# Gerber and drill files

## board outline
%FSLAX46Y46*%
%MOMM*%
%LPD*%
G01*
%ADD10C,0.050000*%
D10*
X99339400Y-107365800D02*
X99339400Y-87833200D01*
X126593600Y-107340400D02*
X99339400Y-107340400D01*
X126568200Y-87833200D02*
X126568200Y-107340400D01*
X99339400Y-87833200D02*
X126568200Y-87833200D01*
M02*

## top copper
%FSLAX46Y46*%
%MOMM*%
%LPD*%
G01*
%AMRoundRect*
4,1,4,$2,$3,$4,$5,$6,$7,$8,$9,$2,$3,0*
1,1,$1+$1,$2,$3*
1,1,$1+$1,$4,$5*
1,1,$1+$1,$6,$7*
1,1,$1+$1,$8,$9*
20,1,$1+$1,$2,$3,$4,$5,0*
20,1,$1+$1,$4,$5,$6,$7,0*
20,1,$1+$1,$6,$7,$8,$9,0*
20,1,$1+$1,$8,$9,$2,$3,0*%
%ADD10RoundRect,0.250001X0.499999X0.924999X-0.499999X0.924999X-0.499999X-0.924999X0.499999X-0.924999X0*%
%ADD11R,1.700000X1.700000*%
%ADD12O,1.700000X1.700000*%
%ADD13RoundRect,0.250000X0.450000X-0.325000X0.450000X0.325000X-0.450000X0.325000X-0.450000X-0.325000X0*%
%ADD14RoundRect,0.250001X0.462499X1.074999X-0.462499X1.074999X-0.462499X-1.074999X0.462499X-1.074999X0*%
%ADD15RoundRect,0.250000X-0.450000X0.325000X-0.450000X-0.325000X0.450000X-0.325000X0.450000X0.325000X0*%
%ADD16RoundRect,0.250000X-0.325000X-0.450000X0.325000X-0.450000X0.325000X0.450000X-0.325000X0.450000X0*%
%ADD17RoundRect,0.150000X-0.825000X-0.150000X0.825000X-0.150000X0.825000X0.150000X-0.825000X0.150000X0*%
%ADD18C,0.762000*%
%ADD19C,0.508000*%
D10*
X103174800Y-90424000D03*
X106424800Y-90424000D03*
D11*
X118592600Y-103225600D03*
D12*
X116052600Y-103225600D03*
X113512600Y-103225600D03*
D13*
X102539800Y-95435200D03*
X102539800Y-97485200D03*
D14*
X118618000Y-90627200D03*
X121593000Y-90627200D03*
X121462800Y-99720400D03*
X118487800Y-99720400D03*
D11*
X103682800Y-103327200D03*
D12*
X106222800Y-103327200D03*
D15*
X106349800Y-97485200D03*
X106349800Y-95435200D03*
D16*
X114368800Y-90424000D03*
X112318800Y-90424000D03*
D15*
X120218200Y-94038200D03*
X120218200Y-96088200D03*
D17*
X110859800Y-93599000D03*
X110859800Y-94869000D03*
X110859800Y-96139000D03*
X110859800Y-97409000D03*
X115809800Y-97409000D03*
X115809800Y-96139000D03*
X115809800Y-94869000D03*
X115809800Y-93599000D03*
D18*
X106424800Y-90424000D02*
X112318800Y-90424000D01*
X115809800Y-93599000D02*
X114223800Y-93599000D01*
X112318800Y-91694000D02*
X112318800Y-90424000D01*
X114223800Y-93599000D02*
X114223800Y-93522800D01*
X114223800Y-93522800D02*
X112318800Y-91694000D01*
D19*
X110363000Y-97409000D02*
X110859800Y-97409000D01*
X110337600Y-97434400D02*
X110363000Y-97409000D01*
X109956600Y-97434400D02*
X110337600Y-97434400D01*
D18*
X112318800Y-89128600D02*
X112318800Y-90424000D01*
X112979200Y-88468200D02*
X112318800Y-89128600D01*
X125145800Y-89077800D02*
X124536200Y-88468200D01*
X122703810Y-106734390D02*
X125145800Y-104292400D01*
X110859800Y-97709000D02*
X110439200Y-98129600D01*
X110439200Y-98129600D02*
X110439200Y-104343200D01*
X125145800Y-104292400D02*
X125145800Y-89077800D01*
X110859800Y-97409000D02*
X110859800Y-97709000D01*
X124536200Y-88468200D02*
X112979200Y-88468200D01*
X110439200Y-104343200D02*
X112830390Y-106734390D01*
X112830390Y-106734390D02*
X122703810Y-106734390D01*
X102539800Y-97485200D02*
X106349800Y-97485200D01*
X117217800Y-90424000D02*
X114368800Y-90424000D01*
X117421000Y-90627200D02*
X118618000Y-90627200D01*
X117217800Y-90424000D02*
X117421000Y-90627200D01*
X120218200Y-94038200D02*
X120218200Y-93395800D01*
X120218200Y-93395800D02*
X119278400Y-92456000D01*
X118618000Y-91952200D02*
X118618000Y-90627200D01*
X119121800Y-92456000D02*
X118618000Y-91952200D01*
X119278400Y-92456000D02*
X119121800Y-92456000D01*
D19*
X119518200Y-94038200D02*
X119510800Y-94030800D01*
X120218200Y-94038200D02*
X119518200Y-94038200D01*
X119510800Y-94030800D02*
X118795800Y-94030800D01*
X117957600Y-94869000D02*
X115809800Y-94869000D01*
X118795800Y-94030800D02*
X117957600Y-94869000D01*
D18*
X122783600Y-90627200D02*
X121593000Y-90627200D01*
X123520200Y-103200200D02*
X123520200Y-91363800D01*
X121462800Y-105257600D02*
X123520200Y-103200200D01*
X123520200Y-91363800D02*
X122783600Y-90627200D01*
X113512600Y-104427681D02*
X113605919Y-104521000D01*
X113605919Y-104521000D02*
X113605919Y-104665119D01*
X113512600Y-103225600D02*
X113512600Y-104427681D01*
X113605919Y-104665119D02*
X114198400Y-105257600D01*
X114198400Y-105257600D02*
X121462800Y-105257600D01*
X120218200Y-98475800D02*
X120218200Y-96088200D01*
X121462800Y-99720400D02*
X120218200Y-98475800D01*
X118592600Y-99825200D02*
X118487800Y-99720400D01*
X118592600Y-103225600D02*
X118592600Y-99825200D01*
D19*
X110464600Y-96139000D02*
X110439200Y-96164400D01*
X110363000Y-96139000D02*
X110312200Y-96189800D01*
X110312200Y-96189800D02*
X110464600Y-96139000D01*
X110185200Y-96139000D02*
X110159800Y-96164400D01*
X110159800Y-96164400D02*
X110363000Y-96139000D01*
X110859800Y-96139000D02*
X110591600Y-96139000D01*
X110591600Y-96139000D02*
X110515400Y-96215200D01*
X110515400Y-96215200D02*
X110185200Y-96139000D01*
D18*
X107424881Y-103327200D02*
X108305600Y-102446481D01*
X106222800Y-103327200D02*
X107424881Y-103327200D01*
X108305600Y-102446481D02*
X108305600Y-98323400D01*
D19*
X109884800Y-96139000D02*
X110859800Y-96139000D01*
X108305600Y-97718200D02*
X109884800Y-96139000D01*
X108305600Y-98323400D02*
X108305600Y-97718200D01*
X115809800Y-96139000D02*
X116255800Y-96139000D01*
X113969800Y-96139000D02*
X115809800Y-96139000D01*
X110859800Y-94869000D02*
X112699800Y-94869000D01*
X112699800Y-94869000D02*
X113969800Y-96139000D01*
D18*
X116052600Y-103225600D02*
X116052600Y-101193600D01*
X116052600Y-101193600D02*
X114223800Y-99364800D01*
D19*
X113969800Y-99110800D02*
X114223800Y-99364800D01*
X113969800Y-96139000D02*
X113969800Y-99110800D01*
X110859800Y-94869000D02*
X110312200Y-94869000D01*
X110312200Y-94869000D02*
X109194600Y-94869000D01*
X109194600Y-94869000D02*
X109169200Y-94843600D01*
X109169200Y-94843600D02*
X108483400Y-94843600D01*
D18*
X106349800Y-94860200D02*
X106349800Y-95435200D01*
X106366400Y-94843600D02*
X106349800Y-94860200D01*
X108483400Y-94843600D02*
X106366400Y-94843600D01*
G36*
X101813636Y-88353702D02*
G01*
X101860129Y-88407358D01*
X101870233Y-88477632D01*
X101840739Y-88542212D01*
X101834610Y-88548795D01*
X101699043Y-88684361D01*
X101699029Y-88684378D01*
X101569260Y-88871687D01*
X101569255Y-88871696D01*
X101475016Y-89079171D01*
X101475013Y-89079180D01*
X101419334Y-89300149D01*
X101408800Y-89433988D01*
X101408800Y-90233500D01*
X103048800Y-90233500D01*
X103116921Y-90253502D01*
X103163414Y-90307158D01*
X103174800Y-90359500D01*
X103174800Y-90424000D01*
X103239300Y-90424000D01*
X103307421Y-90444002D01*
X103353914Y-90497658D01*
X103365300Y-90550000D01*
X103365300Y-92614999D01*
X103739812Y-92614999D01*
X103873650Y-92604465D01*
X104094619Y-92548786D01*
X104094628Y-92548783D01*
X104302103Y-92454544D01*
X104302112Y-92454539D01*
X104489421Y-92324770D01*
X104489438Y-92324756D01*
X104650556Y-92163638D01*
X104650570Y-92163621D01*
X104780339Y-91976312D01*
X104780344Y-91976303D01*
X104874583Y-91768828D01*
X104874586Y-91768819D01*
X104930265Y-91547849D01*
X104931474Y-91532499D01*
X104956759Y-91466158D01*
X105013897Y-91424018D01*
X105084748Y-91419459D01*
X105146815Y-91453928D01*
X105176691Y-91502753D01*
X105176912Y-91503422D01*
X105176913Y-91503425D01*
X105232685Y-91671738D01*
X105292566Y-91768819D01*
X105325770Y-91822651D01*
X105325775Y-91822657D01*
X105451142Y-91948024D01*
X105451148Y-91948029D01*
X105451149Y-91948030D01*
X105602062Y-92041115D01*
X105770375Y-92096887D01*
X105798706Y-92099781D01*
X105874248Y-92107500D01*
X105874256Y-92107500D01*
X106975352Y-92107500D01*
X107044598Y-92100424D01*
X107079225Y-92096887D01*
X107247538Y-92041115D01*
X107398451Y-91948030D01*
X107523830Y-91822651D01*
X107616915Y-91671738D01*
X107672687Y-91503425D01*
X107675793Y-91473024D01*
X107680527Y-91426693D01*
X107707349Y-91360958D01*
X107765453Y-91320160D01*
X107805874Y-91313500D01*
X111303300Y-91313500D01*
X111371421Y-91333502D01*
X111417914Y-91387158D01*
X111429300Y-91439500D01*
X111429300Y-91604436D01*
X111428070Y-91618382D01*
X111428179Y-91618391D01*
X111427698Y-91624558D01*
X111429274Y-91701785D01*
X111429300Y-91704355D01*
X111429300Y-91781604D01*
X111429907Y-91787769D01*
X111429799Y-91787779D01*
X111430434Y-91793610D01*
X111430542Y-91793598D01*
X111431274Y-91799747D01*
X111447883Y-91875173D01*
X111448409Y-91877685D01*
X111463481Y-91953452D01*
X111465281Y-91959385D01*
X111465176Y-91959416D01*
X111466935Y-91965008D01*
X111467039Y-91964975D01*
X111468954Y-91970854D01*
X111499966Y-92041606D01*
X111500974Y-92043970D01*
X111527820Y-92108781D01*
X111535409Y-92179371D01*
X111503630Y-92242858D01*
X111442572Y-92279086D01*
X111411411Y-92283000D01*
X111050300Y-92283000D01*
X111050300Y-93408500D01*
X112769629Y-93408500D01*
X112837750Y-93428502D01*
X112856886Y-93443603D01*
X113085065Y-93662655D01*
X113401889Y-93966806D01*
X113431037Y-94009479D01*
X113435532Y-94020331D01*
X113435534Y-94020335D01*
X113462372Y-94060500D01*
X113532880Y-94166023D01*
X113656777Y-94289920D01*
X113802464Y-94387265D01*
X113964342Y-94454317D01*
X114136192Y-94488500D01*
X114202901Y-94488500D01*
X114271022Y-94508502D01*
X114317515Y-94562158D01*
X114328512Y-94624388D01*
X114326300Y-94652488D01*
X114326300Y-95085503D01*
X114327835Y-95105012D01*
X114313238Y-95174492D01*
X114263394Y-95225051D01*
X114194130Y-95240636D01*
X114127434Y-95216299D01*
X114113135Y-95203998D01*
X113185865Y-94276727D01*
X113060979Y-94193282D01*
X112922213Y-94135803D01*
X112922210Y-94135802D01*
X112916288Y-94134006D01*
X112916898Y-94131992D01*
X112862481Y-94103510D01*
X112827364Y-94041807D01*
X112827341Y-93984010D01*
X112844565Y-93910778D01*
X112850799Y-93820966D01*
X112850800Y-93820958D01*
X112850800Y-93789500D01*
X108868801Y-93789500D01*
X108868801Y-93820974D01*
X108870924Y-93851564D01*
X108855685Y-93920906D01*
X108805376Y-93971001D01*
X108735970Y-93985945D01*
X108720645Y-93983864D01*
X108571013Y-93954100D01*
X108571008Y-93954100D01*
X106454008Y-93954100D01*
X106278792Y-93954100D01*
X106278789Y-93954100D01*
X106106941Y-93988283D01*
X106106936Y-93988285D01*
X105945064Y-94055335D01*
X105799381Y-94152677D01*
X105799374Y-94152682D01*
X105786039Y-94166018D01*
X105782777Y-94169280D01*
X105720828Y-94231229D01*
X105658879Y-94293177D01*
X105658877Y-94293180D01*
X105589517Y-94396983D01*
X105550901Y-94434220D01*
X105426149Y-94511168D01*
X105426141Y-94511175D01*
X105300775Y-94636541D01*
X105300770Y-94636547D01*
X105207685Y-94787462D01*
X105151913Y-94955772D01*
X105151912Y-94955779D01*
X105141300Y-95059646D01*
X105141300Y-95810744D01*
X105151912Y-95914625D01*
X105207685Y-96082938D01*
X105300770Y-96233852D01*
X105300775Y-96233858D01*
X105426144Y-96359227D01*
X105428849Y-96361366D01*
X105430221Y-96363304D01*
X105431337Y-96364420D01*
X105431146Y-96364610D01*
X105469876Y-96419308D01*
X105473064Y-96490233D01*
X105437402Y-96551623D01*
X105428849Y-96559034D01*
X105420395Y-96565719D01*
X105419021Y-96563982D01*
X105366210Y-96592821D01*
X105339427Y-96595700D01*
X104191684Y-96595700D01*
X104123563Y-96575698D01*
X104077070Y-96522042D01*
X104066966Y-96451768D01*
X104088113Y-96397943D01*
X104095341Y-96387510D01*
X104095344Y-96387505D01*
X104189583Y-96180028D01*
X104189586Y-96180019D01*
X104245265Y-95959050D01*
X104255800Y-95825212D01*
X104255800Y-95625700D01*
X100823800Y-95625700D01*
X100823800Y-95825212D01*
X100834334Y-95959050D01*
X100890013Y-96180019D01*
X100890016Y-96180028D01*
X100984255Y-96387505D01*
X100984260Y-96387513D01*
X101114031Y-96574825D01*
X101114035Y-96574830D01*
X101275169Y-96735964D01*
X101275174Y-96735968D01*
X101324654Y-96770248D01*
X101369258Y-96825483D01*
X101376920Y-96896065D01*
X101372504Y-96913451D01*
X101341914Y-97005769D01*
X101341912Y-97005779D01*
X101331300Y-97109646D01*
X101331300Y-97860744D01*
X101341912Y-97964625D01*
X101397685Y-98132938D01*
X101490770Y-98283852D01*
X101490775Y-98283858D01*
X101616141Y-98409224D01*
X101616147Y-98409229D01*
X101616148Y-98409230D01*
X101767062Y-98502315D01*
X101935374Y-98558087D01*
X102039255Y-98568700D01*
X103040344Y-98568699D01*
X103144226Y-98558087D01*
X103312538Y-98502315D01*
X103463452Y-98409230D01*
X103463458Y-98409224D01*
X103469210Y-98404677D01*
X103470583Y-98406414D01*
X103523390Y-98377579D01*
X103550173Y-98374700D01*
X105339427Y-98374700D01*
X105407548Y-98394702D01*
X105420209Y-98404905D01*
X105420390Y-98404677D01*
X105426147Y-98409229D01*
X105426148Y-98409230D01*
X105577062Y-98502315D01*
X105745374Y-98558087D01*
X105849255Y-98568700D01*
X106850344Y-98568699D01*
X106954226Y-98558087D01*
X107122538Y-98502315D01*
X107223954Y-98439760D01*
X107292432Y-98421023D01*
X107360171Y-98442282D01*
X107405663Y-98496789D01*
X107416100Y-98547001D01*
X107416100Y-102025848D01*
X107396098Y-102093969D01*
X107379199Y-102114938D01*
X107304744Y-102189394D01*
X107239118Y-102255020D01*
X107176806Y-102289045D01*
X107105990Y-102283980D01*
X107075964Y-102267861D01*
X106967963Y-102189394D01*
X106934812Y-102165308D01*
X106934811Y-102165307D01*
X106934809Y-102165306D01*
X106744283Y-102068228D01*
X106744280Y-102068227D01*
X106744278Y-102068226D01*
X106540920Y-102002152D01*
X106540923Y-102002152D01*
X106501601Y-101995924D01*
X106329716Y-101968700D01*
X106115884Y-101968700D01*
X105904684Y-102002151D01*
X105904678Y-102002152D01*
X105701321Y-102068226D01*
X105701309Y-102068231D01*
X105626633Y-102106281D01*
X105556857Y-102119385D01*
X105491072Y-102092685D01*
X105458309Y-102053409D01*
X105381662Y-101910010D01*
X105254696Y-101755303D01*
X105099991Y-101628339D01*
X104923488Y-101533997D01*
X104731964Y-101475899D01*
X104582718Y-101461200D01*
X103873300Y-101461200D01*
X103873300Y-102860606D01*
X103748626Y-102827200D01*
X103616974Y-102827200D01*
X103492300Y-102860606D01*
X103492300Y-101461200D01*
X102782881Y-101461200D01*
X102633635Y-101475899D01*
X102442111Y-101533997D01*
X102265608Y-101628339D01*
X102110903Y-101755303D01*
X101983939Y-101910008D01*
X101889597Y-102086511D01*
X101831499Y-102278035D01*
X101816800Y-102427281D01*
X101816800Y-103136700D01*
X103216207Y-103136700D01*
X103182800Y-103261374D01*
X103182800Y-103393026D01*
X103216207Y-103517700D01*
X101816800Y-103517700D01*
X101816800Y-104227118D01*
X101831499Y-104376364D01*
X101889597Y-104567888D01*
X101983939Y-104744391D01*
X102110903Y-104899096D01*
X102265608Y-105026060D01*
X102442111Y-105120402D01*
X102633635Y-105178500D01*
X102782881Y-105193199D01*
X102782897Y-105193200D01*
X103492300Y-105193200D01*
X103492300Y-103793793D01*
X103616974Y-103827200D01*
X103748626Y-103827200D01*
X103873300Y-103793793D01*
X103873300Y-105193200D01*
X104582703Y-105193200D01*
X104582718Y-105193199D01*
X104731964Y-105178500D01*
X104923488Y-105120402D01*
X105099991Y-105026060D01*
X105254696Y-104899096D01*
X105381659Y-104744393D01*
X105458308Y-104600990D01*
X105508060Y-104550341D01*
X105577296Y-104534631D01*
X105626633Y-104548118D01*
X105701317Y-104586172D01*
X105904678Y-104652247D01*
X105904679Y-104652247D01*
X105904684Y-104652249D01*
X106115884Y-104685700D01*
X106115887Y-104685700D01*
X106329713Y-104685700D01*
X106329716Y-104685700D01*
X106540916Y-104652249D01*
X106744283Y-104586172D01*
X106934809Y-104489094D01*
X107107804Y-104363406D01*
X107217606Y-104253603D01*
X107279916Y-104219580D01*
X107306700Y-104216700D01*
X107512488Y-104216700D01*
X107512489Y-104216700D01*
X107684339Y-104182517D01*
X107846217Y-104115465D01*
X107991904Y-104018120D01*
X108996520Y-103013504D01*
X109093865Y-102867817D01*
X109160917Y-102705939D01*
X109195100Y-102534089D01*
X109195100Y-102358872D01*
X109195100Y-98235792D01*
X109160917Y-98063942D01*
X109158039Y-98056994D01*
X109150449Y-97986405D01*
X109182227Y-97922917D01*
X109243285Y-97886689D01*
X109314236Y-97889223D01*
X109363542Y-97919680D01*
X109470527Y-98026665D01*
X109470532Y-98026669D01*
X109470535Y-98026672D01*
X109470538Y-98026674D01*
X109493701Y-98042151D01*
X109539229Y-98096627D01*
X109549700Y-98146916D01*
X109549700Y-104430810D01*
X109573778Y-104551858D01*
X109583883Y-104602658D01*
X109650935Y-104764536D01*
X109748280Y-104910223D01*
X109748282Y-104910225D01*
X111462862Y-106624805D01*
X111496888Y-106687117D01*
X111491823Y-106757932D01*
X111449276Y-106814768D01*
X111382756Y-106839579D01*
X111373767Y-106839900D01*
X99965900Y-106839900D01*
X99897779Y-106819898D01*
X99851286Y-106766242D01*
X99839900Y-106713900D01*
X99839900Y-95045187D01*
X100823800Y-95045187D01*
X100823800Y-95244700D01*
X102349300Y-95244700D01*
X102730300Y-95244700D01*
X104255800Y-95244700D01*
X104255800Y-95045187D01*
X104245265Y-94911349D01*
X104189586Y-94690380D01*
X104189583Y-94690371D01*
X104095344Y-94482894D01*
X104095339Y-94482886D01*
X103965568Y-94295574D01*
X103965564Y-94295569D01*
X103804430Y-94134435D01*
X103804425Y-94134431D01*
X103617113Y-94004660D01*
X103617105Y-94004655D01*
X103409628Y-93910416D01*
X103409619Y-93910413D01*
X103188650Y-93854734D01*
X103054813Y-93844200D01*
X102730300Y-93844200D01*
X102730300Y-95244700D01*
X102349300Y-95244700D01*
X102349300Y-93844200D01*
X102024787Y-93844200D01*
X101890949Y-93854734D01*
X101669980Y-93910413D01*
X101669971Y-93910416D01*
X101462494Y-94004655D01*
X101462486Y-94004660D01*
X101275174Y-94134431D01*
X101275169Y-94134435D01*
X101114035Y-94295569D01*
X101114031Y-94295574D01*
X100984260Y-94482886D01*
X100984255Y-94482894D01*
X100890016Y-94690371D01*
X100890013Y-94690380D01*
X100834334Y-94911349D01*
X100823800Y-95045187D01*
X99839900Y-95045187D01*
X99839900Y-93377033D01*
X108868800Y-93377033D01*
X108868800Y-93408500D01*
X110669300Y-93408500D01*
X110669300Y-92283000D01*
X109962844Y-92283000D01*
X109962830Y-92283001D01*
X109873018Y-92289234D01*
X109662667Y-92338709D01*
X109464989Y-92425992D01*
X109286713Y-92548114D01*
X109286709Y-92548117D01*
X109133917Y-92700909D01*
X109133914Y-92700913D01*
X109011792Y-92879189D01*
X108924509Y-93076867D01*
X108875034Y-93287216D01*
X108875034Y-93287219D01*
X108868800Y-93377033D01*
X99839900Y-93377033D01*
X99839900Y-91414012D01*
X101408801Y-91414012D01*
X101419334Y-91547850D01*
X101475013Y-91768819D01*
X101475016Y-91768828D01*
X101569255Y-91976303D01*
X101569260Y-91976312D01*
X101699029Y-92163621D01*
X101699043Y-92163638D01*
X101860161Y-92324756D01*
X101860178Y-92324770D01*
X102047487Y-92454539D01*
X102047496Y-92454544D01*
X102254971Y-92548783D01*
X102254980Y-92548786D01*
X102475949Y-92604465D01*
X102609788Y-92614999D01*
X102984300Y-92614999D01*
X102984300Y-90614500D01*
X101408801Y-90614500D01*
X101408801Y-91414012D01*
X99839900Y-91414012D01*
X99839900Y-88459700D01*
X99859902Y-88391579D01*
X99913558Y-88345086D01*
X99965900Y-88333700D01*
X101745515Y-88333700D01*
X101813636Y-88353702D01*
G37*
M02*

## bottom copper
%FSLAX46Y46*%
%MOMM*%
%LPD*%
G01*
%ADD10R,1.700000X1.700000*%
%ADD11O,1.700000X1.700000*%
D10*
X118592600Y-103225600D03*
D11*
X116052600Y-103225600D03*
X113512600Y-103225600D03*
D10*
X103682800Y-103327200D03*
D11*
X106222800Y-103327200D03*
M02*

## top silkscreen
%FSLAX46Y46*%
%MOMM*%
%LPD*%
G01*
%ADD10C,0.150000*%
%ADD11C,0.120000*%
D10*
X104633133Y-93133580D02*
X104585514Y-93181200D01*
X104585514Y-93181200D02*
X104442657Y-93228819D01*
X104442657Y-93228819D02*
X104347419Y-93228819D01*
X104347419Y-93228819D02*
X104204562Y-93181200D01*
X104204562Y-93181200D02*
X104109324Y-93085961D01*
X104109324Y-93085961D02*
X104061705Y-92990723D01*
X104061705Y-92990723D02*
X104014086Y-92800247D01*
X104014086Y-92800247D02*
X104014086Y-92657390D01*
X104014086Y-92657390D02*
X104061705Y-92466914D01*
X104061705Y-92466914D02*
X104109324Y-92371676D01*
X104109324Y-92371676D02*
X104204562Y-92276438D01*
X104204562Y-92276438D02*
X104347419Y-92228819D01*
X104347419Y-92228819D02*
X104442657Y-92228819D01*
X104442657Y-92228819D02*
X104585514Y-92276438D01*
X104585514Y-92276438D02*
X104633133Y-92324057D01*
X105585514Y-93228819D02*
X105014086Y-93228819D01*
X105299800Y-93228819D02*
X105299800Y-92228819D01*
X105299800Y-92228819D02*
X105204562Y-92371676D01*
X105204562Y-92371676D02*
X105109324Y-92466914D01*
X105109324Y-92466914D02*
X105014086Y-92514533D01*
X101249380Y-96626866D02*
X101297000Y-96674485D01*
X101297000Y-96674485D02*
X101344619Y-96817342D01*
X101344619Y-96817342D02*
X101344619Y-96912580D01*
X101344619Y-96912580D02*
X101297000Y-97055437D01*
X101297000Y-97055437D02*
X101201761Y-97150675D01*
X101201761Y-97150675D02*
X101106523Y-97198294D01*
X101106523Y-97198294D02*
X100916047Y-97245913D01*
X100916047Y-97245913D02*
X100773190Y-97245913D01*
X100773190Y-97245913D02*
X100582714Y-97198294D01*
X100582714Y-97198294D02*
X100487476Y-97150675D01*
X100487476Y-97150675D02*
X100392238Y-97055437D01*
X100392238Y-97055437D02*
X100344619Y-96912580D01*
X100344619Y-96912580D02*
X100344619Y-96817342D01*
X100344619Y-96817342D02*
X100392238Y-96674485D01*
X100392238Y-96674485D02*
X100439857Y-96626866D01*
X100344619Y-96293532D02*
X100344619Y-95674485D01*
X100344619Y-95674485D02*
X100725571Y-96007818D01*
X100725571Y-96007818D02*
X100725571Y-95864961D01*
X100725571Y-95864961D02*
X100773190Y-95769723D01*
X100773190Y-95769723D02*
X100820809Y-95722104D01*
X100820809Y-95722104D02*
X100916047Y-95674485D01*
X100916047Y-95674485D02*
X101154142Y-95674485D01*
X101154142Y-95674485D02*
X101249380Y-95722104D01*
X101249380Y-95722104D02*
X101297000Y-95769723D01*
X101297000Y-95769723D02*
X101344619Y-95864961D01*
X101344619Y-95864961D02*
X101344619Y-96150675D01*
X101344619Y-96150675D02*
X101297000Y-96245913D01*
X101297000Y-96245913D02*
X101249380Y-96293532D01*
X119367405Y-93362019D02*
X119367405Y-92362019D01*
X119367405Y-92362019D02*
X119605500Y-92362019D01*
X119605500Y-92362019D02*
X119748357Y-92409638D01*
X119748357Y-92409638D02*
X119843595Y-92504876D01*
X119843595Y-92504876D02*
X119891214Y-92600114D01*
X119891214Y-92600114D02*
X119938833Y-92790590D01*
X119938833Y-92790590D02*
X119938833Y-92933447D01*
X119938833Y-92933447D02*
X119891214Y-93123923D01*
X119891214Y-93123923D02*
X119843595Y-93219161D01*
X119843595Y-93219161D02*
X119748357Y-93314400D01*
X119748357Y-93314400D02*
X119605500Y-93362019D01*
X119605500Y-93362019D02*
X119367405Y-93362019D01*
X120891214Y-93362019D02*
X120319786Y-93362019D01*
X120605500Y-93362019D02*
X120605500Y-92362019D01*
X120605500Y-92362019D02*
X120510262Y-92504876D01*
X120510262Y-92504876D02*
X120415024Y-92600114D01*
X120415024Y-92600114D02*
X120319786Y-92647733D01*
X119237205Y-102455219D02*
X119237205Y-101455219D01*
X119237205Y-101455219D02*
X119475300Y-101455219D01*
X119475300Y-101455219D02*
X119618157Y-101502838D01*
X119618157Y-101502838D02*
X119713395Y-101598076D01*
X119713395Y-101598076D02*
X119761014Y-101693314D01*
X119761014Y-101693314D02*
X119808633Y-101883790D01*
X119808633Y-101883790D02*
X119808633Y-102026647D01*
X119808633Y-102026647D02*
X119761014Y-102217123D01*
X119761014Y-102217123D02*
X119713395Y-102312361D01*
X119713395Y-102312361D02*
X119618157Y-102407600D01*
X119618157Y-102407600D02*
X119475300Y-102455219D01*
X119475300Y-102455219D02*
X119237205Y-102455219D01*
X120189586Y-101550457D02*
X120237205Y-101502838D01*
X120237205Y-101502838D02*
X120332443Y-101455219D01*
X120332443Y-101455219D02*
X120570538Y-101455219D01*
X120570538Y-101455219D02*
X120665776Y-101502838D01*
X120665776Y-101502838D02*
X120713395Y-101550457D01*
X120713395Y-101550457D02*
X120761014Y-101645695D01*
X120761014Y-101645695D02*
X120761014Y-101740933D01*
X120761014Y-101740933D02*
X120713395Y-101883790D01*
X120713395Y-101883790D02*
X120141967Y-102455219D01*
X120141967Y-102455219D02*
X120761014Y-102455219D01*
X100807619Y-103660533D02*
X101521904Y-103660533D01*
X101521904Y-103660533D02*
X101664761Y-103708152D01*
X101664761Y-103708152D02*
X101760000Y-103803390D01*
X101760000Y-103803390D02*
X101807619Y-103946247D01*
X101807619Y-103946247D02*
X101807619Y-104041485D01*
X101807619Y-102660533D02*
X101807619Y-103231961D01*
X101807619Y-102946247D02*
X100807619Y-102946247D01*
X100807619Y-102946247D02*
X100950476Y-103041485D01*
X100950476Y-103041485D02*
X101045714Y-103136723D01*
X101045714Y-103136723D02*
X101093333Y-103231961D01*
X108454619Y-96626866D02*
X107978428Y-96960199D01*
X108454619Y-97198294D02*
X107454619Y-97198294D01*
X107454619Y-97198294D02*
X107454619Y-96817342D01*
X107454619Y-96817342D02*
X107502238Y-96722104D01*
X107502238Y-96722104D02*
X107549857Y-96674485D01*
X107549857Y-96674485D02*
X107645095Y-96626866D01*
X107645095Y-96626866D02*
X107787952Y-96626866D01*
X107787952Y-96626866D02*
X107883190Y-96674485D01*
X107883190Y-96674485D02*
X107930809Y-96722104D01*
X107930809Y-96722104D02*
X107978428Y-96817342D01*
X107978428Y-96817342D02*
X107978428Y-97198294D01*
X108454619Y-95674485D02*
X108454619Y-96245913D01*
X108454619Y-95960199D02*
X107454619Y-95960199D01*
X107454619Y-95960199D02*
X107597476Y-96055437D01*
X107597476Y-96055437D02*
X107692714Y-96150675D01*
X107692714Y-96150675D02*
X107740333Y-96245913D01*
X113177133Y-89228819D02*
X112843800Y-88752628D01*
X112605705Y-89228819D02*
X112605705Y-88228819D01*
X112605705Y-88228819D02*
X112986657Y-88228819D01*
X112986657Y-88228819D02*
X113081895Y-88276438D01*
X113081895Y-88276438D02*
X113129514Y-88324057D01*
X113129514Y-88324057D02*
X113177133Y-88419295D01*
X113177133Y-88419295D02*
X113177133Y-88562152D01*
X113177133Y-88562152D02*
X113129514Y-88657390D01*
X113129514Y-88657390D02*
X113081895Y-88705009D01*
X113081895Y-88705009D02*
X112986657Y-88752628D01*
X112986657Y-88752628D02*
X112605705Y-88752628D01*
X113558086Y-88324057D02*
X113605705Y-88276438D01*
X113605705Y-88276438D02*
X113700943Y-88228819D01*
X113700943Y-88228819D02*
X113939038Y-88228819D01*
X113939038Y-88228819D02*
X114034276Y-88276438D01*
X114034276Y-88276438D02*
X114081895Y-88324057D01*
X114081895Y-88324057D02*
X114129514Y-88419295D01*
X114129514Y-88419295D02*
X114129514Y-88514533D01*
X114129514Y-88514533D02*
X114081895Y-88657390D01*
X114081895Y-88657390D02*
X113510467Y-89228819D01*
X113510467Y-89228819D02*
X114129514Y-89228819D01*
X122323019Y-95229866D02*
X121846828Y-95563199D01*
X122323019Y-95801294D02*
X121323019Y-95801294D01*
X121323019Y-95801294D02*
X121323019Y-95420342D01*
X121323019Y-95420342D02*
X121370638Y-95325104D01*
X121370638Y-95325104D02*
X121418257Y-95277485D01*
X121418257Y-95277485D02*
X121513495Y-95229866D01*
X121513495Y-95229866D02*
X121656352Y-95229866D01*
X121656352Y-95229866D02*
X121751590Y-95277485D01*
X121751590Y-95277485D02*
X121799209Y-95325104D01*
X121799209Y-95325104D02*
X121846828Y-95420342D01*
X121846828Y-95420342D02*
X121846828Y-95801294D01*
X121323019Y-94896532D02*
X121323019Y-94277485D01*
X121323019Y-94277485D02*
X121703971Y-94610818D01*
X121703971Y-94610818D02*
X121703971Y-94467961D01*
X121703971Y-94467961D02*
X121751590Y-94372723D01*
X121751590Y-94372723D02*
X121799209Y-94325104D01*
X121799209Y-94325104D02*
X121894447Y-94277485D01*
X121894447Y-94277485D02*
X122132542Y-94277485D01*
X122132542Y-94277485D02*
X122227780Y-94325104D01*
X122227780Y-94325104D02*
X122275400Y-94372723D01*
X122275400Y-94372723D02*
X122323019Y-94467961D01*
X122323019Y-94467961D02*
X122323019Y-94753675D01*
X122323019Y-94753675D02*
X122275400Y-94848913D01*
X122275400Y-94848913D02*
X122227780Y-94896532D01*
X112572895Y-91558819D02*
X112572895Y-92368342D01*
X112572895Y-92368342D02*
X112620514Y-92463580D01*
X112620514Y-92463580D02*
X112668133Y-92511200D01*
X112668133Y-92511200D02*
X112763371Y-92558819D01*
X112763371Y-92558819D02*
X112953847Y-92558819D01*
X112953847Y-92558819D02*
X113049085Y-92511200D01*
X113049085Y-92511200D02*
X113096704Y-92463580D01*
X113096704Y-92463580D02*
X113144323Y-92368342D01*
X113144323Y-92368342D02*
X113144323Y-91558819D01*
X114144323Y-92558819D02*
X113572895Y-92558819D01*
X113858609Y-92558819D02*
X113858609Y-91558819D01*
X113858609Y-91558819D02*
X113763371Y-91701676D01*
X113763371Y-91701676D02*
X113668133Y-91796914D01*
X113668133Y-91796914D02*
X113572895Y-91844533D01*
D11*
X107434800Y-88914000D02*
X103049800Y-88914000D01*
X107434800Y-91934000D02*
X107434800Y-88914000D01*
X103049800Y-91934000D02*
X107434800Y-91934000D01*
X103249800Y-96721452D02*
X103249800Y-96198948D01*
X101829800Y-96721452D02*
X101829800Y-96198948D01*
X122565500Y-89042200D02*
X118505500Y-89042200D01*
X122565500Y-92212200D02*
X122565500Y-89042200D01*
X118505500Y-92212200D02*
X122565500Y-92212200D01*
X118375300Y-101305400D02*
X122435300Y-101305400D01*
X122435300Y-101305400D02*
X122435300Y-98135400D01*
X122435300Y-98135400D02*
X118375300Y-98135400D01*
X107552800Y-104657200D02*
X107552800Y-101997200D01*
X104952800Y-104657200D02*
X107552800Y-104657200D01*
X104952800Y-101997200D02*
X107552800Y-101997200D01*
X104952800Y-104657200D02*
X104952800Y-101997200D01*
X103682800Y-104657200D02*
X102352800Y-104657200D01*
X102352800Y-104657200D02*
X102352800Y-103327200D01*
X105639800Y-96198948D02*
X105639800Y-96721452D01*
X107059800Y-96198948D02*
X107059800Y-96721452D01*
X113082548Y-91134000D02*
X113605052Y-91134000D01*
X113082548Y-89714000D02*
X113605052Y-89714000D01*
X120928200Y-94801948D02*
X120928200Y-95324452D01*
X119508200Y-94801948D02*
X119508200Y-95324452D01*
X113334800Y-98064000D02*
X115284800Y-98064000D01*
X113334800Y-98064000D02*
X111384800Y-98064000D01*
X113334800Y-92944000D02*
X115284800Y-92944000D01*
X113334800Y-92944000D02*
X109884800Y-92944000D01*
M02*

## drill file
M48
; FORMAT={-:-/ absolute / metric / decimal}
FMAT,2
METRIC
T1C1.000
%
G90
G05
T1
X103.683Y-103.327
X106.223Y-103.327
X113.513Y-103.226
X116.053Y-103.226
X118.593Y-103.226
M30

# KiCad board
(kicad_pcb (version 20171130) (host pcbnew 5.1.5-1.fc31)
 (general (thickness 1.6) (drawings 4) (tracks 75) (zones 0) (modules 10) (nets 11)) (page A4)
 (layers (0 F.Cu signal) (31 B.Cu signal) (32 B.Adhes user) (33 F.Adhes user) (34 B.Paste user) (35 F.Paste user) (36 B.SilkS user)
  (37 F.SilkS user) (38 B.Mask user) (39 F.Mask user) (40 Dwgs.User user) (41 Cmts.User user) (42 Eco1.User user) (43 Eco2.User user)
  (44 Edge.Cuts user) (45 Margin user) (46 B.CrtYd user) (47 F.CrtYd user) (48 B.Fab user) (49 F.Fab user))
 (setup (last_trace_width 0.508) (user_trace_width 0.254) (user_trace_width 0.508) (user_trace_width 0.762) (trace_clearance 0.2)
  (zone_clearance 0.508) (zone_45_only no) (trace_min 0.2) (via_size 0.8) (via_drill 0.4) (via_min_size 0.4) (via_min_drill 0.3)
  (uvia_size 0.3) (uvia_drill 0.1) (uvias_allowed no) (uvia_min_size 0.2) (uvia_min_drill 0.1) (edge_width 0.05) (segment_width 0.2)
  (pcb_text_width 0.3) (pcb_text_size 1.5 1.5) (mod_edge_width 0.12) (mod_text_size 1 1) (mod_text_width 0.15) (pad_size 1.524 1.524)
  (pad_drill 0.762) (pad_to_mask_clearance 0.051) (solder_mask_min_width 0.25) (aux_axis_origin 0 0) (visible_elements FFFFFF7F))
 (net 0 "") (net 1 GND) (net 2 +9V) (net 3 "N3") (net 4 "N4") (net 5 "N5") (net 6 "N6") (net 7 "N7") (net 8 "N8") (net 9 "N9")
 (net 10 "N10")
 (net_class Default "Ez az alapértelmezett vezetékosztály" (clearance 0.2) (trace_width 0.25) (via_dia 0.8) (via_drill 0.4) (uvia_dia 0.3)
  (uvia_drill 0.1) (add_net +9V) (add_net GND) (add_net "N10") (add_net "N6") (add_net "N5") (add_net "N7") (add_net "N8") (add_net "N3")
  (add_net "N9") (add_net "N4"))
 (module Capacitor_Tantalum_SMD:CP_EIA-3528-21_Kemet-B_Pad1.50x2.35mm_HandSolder (layer F.Cu) (at 104.7998 90.424 180)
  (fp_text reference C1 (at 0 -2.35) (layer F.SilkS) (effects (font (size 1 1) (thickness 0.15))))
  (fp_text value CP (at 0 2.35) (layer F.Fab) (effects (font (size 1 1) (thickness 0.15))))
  (fp_line (start -2.635 1.51) (end 1.75 1.51) (layer F.SilkS) (width 0.12))
  (fp_line (start -2.635 -1.51) (end -2.635 1.51) (layer F.SilkS) (width 0.12))
  (fp_line (start 1.75 -1.51) (end -2.635 -1.51) (layer F.SilkS) (width 0.12))
  (pad 2 smd roundrect (at 1.625 0 180) (size 1.5 2.35) (layers F.Cu F.Paste F.Mask) (roundrect_rratio 0.166667) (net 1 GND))
  (pad 1 smd roundrect (at -1.625 0 180) (size 1.5 2.35) (layers F.Cu F.Paste F.Mask) (roundrect_rratio 0.166667) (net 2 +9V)))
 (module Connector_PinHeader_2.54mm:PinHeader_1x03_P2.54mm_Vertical (layer B.Cu) (at 118.5926 103.2256 90)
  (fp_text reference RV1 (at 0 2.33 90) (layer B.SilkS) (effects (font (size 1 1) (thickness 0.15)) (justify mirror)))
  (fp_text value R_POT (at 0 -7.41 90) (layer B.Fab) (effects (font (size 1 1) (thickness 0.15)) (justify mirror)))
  (pad 1 thru_hole rect (at 0 0 90) (size 1.7 1.7) (drill 1) (layers *.Cu *.Mask) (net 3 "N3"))
  (pad 2 thru_hole oval (at 0 -2.54 90) (size 1.7 1.7) (drill 1) (layers *.Cu *.Mask) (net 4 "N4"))
  (pad 3 thru_hole oval (at 0 -5.08 90) (size 1.7 1.7) (drill 1) (layers *.Cu *.Mask) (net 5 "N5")))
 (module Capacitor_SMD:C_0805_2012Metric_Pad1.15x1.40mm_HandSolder (layer F.Cu) (at 102.5398 96.4602 90)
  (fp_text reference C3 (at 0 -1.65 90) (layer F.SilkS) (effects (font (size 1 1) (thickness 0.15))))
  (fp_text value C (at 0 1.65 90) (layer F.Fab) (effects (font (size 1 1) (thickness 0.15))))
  (fp_line (start -0.261252 0.71) (end 0.261252 0.71) (layer F.SilkS) (width 0.12))
  (fp_line (start -0.261252 -0.71) (end 0.261252 -0.71) (layer F.SilkS) (width 0.12))
  (pad 2 smd roundrect (at 1.025 0 90) (size 1.15 1.4) (layers F.Cu F.Paste F.Mask) (roundrect_rratio 0.217391) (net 1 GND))
  (pad 1 smd roundrect (at -1.025 0 90) (size 1.15 1.4) (layers F.Cu F.Paste F.Mask) (roundrect_rratio 0.217391) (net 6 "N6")))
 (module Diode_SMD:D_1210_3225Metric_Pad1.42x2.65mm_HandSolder (layer F.Cu) (at 120.1055 90.6272 180)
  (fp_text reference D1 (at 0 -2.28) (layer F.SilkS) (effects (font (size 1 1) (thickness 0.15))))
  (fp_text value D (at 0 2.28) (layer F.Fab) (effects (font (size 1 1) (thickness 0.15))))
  (fp_line (start -2.46 1.585) (end 1.6 1.585) (layer F.SilkS) (width 0.12))
  (fp_line (start -2.46 -1.585) (end -2.46 1.585) (layer F.SilkS) (width 0.12))
  (fp_line (start 1.6 -1.585) (end -2.46 -1.585) (layer F.SilkS) (width 0.12))
  (pad 2 smd roundrect (at 1.4875 0 180) (size 1.425 2.65) (layers F.Cu F.Paste F.Mask) (roundrect_rratio 0.175439) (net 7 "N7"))
  (pad 1 smd roundrect (at -1.4875 0 180) (size 1.425 2.65) (layers F.Cu F.Paste F.Mask) (roundrect_rratio 0.175439) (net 5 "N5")))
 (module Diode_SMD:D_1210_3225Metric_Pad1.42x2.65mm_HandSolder (layer F.Cu) (at 119.9753 99.7204 180)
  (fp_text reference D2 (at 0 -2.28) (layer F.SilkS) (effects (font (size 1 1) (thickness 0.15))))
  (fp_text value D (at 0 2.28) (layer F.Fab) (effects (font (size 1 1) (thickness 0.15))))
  (fp_line (start 1.6 -1.585) (end -2.46 -1.585) (layer F.SilkS) (width 0.12))
  (fp_line (start -2.46 -1.585) (end -2.46 1.585) (layer F.SilkS) (width 0.12))
  (fp_line (start -2.46 1.585) (end 1.6 1.585) (layer F.SilkS) (width 0.12))
  (pad 1 smd roundrect (at -1.4875 0 180) (size 1.425 2.65) (layers F.Cu F.Paste F.Mask) (roundrect_rratio 0.175439) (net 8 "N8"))
  (pad 2 smd roundrect (at 1.4875 0 180) (size 1.425 2.65) (layers F.Cu F.Paste F.Mask) (roundrect_rratio 0.175439) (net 3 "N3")))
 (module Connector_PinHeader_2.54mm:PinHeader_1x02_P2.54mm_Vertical (layer F.Cu) (at 103.6828 103.3272 90)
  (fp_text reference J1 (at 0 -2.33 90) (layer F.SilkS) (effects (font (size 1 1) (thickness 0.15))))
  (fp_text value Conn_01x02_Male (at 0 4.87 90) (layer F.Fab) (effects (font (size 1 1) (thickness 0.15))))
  (fp_line (start -1.33 3.87) (end 1.33 3.87) (layer F.SilkS) (width 0.12))
  (fp_line (start -1.33 1.27) (end -1.33 3.87) (layer F.SilkS) (width 0.12))
  (fp_line (start 1.33 1.27) (end 1.33 3.87) (layer F.SilkS) (width 0.12))
  (fp_line (start -1.33 1.27) (end 1.33 1.27) (layer F.SilkS) (width 0.12))
  (fp_line (start -1.33 0) (end -1.33 -1.33) (layer F.SilkS) (width 0.12))
  (fp_line (start -1.33 -1.33) (end 0 -1.33) (layer F.SilkS) (width 0.12))
  (pad 1 thru_hole rect (at 0 0 90) (size 1.7 1.7) (drill 1) (layers *.Cu *.Mask) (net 1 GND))
  (pad 2 thru_hole oval (at 0 2.54 90) (size 1.7 1.7) (drill 1) (layers *.Cu *.Mask) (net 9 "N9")))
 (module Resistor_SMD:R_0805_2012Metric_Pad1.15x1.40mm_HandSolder (layer F.Cu) (at 106.3498 96.4602 270)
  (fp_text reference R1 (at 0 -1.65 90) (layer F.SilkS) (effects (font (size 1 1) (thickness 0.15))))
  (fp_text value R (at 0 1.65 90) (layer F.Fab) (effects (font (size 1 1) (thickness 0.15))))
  (fp_line (start -0.261252 0.71) (end 0.261252 0.71) (layer F.SilkS) (width 0.12))
  (fp_line (start -0.261252 -0.71) (end 0.261252 -0.71) (layer F.SilkS) (width 0.12))
  (pad 2 smd roundrect (at 1.025 0 270) (size 1.15 1.4) (layers F.Cu F.Paste F.Mask) (roundrect_rratio 0.217391) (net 6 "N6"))
  (pad 1 smd roundrect (at -1.025 0 270) (size 1.15 1.4) (layers F.Cu F.Paste F.Mask) (roundrect_rratio 0.217391) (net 4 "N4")))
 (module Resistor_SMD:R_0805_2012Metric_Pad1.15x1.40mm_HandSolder (layer F.Cu) (at 113.3438 90.424)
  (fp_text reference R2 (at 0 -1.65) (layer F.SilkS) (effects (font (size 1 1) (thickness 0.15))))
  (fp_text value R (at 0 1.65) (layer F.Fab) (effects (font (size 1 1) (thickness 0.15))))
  (fp_line (start -0.261252 0.71) (end 0.261252 0.71) (layer F.SilkS) (width 0.12))
  (fp_line (start -0.261252 -0.71) (end 0.261252 -0.71) (layer F.SilkS) (width 0.12))
  (pad 2 smd roundrect (at 1.025 0) (size 1.15 1.4) (layers F.Cu F.Paste F.Mask) (roundrect_rratio 0.217391) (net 7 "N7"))
  (pad 1 smd roundrect (at -1.025 0) (size 1.15 1.4) (layers F.Cu F.Paste F.Mask) (roundrect_rratio 0.217391) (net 2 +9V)))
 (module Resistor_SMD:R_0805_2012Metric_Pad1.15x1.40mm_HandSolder (layer F.Cu) (at 120.2182 95.0632 270)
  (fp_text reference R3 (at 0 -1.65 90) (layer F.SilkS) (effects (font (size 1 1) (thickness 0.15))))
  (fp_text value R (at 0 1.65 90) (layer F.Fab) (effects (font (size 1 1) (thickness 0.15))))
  (fp_line (start -0.261252 -0.71) (end 0.261252 -0.71) (layer F.SilkS) (width 0.12))
  (fp_line (start -0.261252 0.71) (end 0.261252 0.71) (layer F.SilkS) (width 0.12))
  (pad 1 smd roundrect (at -1.025 0 270) (size 1.15 1.4) (layers F.Cu F.Paste F.Mask) (roundrect_rratio 0.217391) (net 7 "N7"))
  (pad 2 smd roundrect (at 1.025 0 270) (size 1.15 1.4) (layers F.Cu F.Paste F.Mask) (roundrect_rratio 0.217391) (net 8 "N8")))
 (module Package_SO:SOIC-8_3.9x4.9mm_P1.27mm (layer F.Cu) (at 113.3348 95.504)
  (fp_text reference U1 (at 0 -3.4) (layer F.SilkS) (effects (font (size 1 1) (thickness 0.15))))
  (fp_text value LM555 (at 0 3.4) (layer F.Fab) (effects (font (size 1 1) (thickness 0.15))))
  (fp_line (start 0 2.56) (end 1.95 2.56) (layer F.SilkS) (width 0.12))
  (fp_line (start 0 2.56) (end -1.95 2.56) (layer F.SilkS) (width 0.12))
  (fp_line (start 0 -2.56) (end 1.95 -2.56) (layer F.SilkS) (width 0.12))
  (fp_line (start 0 -2.56) (end -3.45 -2.56) (layer F.SilkS) (width 0.12))
  (pad 1 smd roundrect (at -2.475 -1.905) (size 1.95 0.6) (layers F.Cu F.Paste F.Mask) (roundrect_rratio 0.25) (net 1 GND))
  (pad 2 smd roundrect (at -2.475 -0.635) (size 1.95 0.6) (layers F.Cu F.Paste F.Mask) (roundrect_rratio 0.25) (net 4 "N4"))
  (pad 3 smd roundrect (at -2.475 0.635) (size 1.95 0.6) (layers F.Cu F.Paste F.Mask) (roundrect_rratio 0.25) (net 9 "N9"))
  (pad 4 smd roundrect (at -2.475 1.905) (size 1.95 0.6) (layers F.Cu F.Paste F.Mask) (roundrect_rratio 0.25) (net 2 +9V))
  (pad 5 smd roundrect (at 2.475 1.905) (size 1.95 0.6) (layers F.Cu F.Paste F.Mask) (roundrect_rratio 0.25) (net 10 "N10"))
  (pad 6 smd roundrect (at 2.475 0.635) (size 1.95 0.6) (layers F.Cu F.Paste F.Mask) (roundrect_rratio 0.25) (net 4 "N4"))
  (pad 7 smd roundrect (at 2.475 -0.635) (size 1.95 0.6) (layers F.Cu F.Paste F.Mask) (roundrect_rratio 0.25) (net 7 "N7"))
  (pad 8 smd roundrect (at 2.475 -1.905) (size 1.95 0.6) (layers F.Cu F.Paste F.Mask) (roundrect_rratio 0.25) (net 2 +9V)))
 (gr_line (start 99.3394 107.3658) (end 99.3394 87.8332) (layer Edge.Cuts) (width 0.05))
 (gr_line (start 126.5936 107.3404) (end 99.3394 107.3404) (layer Edge.Cuts) (width 0.05))
 (gr_line (start 126.5682 87.8332) (end 126.5682 107.3404) (layer Edge.Cuts) (width 0.05))
 (gr_line (start 99.3394 87.8332) (end 126.5682 87.8332) (layer Edge.Cuts) (width 0.05))
 (segment (start 106.4248 90.424) (end 112.3188 90.424) (width 0.762) (layer F.Cu) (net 2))
 (segment (start 115.8098 93.599) (end 114.2238 93.599) (width 0.762) (layer F.Cu) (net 2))
 (segment (start 112.3188 91.694) (end 112.3188 90.424) (width 0.762) (layer F.Cu) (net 2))
 (segment (start 114.2238 93.599) (end 114.2238 93.5228) (width 0.762) (layer F.Cu) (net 2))
 (segment (start 114.2238 93.5228) (end 112.3188 91.694) (width 0.762) (layer F.Cu) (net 2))
 (segment (start 110.363 97.409) (end 110.8598 97.409) (width 0.508) (layer F.Cu) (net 2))
 (segment (start 110.3376 97.4344) (end 110.363 97.409) (width 0.508) (layer F.Cu) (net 2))
 (segment (start 109.9566 97.4344) (end 110.3376 97.4344) (width 0.508) (layer F.Cu) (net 2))
 (segment (start 112.3188 89.1286) (end 112.3188 90.424) (width 0.762) (layer F.Cu) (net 2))
 (segment (start 112.9792 88.4682) (end 112.3188 89.1286) (width 0.762) (layer F.Cu) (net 2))
 (segment (start 125.1458 89.0778) (end 124.5362 88.4682) (width 0.762) (layer F.Cu) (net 2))
 (segment (start 122.70381 106.73439) (end 125.1458 104.2924) (width 0.762) (layer F.Cu) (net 2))
 (segment (start 110.8598 97.709) (end 110.4392 98.1296) (width 0.762) (layer F.Cu) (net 2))
 (segment (start 110.4392 98.1296) (end 110.4392 104.3432) (width 0.762) (layer F.Cu) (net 2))
 (segment (start 125.1458 104.2924) (end 125.1458 89.0778) (width 0.762) (layer F.Cu) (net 2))
 (segment (start 110.8598 97.409) (end 110.8598 97.709) (width 0.762) (layer F.Cu) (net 2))
 (segment (start 124.5362 88.4682) (end 112.9792 88.4682) (width 0.762) (layer F.Cu) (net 2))
 (segment (start 110.4392 104.3432) (end 112.83039 106.73439) (width 0.762) (layer F.Cu) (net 2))
 (segment (start 112.83039 106.73439) (end 122.70381 106.73439) (width 0.762) (layer F.Cu) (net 2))
 (segment (start 102.5398 97.4852) (end 106.3498 97.4852) (width 0.762) (layer F.Cu) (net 6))
 (segment (start 117.2178 90.424) (end 114.3688 90.424) (width 0.762) (layer F.Cu) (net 7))
 (segment (start 117.421 90.6272) (end 118.618 90.6272) (width 0.762) (layer F.Cu) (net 7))
 (segment (start 117.2178 90.424) (end 117.421 90.6272) (width 0.762) (layer F.Cu) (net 7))
 (segment (start 120.2182 94.0382) (end 120.2182 93.3958) (width 0.762) (layer F.Cu) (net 7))
 (segment (start 120.2182 93.3958) (end 119.2784 92.456) (width 0.762) (layer F.Cu) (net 7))
 (segment (start 118.618 91.9522) (end 118.618 90.6272) (width 0.762) (layer F.Cu) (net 7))
 (segment (start 119.1218 92.456) (end 118.618 91.9522) (width 0.762) (layer F.Cu) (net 7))
 (segment (start 119.2784 92.456) (end 119.1218 92.456) (width 0.762) (layer F.Cu) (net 7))
 (segment (start 119.5182 94.0382) (end 119.5108 94.0308) (width 0.508) (layer F.Cu) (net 7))
 (segment (start 120.2182 94.0382) (end 119.5182 94.0382) (width 0.508) (layer F.Cu) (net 7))
 (segment (start 119.5108 94.0308) (end 118.7958 94.0308) (width 0.508) (layer F.Cu) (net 7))
 (segment (start 117.9576 94.869) (end 115.8098 94.869) (width 0.508) (layer F.Cu) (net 7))
 (segment (start 118.7958 94.0308) (end 117.9576 94.869) (width 0.508) (layer F.Cu) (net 7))
 (segment (start 122.7836 90.6272) (end 121.593 90.6272) (width 0.762) (layer F.Cu) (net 5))
 (segment (start 123.5202 103.2002) (end 123.5202 91.3638) (width 0.762) (layer F.Cu) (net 5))
 (segment (start 121.4628 105.2576) (end 123.5202 103.2002) (width 0.762) (layer F.Cu) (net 5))
 (segment (start 123.5202 91.3638) (end 122.7836 90.6272) (width 0.762) (layer F.Cu) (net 5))
 (segment (start 113.5126 104.427681) (end 113.605919 104.521) (width 0.762) (layer F.Cu) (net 5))
 (segment (start 113.605919 104.521) (end 113.605919 104.665119) (width 0.762) (layer F.Cu) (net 5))
 (segment (start 113.5126 103.2256) (end 113.5126 104.427681) (width 0.762) (layer F.Cu) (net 5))
 (segment (start 113.605919 104.665119) (end 114.1984 105.2576) (width 0.762) (layer F.Cu) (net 5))
 (segment (start 114.1984 105.2576) (end 121.4628 105.2576) (width 0.762) (layer F.Cu) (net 5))
 (segment (start 120.2182 98.4758) (end 120.2182 96.0882) (width 0.762) (layer F.Cu) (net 8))
 (segment (start 121.4628 99.7204) (end 120.2182 98.4758) (width 0.762) (layer F.Cu) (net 8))
 (segment (start 118.5926 99.8252) (end 118.4878 99.7204) (width 0.762) (layer F.Cu) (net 3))
 (segment (start 118.5926 103.2256) (end 118.5926 99.8252) (width 0.762) (layer F.Cu) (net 3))
 (segment (start 110.4646 96.139) (end 110.4392 96.1644) (width 0.508) (layer F.Cu) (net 9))
 (segment (start 110.363 96.139) (end 110.3122 96.1898) (width 0.508) (layer F.Cu) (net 9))
 (segment (start 110.3122 96.1898) (end 110.4646 96.139) (width 0.508) (layer F.Cu) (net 9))
 (segment (start 110.1852 96.139) (end 110.1598 96.1644) (width 0.508) (layer F.Cu) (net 9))
 (segment (start 110.1598 96.1644) (end 110.363 96.139) (width 0.508) (layer F.Cu) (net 9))
 (segment (start 110.8598 96.139) (end 110.5916 96.139) (width 0.508) (layer F.Cu) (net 9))
 (segment (start 110.5916 96.139) (end 110.5154 96.2152) (width 0.508) (layer F.Cu) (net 9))
 (segment (start 110.5154 96.2152) (end 110.1852 96.139) (width 0.508) (layer F.Cu) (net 9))
 (segment (start 107.424881 103.3272) (end 108.3056 102.446481) (width 0.762) (layer F.Cu) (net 9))
 (segment (start 106.2228 103.3272) (end 107.424881 103.3272) (width 0.762) (layer F.Cu) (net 9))
 (segment (start 108.3056 102.446481) (end 108.3056 98.3234) (width 0.762) (layer F.Cu) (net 9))
 (segment (start 109.8848 96.139) (end 110.8598 96.139) (width 0.508) (layer F.Cu) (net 9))
 (segment (start 108.3056 97.7182) (end 109.8848 96.139) (width 0.508) (layer F.Cu) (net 9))
 (segment (start 108.3056 98.3234) (end 108.3056 97.7182) (width 0.508) (layer F.Cu) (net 9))
 (segment (start 115.8098 96.139) (end 116.2558 96.139) (width 0.508) (layer F.Cu) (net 4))
 (segment (start 113.9698 96.139) (end 115.8098 96.139) (width 0.508) (layer F.Cu) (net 4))
 (segment (start 110.8598 94.869) (end 112.6998 94.869) (width 0.508) (layer F.Cu) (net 4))
 (segment (start 112.6998 94.869) (end 113.9698 96.139) (width 0.508) (layer F.Cu) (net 4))
 (segment (start 116.0526 103.2256) (end 116.0526 101.1936) (width 0.762) (layer F.Cu) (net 4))
 (segment (start 116.0526 101.1936) (end 114.2238 99.3648) (width 0.762) (layer F.Cu) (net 4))
 (segment (start 113.9698 99.1108) (end 114.2238 99.3648) (width 0.508) (layer F.Cu) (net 4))
 (segment (start 113.9698 96.139) (end 113.9698 99.1108) (width 0.508) (layer F.Cu) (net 4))
 (segment (start 110.8598 94.869) (end 110.3122 94.869) (width 0.508) (layer F.Cu) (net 4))
 (segment (start 110.3122 94.869) (end 109.1946 94.869) (width 0.508) (layer F.Cu) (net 4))
 (segment (start 109.1946 94.869) (end 109.1692 94.8436) (width 0.508) (layer F.Cu) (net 4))
 (segment (start 109.1692 94.8436) (end 108.4834 94.8436) (width 0.508) (layer F.Cu) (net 4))
 (segment (start 106.3498 94.8602) (end 106.3498 95.4352) (width 0.762) (layer F.Cu) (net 4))
 (segment (start 106.3664 94.8436) (end 106.3498 94.8602) (width 0.762) (layer F.Cu) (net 4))
 (segment (start 108.4834 94.8436) (end 106.3664 94.8436) (width 0.762) (layer F.Cu) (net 4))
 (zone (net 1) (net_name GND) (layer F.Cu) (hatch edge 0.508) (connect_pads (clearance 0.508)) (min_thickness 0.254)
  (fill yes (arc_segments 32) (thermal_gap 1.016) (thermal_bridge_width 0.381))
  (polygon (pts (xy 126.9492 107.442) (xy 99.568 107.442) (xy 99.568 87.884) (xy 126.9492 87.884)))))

